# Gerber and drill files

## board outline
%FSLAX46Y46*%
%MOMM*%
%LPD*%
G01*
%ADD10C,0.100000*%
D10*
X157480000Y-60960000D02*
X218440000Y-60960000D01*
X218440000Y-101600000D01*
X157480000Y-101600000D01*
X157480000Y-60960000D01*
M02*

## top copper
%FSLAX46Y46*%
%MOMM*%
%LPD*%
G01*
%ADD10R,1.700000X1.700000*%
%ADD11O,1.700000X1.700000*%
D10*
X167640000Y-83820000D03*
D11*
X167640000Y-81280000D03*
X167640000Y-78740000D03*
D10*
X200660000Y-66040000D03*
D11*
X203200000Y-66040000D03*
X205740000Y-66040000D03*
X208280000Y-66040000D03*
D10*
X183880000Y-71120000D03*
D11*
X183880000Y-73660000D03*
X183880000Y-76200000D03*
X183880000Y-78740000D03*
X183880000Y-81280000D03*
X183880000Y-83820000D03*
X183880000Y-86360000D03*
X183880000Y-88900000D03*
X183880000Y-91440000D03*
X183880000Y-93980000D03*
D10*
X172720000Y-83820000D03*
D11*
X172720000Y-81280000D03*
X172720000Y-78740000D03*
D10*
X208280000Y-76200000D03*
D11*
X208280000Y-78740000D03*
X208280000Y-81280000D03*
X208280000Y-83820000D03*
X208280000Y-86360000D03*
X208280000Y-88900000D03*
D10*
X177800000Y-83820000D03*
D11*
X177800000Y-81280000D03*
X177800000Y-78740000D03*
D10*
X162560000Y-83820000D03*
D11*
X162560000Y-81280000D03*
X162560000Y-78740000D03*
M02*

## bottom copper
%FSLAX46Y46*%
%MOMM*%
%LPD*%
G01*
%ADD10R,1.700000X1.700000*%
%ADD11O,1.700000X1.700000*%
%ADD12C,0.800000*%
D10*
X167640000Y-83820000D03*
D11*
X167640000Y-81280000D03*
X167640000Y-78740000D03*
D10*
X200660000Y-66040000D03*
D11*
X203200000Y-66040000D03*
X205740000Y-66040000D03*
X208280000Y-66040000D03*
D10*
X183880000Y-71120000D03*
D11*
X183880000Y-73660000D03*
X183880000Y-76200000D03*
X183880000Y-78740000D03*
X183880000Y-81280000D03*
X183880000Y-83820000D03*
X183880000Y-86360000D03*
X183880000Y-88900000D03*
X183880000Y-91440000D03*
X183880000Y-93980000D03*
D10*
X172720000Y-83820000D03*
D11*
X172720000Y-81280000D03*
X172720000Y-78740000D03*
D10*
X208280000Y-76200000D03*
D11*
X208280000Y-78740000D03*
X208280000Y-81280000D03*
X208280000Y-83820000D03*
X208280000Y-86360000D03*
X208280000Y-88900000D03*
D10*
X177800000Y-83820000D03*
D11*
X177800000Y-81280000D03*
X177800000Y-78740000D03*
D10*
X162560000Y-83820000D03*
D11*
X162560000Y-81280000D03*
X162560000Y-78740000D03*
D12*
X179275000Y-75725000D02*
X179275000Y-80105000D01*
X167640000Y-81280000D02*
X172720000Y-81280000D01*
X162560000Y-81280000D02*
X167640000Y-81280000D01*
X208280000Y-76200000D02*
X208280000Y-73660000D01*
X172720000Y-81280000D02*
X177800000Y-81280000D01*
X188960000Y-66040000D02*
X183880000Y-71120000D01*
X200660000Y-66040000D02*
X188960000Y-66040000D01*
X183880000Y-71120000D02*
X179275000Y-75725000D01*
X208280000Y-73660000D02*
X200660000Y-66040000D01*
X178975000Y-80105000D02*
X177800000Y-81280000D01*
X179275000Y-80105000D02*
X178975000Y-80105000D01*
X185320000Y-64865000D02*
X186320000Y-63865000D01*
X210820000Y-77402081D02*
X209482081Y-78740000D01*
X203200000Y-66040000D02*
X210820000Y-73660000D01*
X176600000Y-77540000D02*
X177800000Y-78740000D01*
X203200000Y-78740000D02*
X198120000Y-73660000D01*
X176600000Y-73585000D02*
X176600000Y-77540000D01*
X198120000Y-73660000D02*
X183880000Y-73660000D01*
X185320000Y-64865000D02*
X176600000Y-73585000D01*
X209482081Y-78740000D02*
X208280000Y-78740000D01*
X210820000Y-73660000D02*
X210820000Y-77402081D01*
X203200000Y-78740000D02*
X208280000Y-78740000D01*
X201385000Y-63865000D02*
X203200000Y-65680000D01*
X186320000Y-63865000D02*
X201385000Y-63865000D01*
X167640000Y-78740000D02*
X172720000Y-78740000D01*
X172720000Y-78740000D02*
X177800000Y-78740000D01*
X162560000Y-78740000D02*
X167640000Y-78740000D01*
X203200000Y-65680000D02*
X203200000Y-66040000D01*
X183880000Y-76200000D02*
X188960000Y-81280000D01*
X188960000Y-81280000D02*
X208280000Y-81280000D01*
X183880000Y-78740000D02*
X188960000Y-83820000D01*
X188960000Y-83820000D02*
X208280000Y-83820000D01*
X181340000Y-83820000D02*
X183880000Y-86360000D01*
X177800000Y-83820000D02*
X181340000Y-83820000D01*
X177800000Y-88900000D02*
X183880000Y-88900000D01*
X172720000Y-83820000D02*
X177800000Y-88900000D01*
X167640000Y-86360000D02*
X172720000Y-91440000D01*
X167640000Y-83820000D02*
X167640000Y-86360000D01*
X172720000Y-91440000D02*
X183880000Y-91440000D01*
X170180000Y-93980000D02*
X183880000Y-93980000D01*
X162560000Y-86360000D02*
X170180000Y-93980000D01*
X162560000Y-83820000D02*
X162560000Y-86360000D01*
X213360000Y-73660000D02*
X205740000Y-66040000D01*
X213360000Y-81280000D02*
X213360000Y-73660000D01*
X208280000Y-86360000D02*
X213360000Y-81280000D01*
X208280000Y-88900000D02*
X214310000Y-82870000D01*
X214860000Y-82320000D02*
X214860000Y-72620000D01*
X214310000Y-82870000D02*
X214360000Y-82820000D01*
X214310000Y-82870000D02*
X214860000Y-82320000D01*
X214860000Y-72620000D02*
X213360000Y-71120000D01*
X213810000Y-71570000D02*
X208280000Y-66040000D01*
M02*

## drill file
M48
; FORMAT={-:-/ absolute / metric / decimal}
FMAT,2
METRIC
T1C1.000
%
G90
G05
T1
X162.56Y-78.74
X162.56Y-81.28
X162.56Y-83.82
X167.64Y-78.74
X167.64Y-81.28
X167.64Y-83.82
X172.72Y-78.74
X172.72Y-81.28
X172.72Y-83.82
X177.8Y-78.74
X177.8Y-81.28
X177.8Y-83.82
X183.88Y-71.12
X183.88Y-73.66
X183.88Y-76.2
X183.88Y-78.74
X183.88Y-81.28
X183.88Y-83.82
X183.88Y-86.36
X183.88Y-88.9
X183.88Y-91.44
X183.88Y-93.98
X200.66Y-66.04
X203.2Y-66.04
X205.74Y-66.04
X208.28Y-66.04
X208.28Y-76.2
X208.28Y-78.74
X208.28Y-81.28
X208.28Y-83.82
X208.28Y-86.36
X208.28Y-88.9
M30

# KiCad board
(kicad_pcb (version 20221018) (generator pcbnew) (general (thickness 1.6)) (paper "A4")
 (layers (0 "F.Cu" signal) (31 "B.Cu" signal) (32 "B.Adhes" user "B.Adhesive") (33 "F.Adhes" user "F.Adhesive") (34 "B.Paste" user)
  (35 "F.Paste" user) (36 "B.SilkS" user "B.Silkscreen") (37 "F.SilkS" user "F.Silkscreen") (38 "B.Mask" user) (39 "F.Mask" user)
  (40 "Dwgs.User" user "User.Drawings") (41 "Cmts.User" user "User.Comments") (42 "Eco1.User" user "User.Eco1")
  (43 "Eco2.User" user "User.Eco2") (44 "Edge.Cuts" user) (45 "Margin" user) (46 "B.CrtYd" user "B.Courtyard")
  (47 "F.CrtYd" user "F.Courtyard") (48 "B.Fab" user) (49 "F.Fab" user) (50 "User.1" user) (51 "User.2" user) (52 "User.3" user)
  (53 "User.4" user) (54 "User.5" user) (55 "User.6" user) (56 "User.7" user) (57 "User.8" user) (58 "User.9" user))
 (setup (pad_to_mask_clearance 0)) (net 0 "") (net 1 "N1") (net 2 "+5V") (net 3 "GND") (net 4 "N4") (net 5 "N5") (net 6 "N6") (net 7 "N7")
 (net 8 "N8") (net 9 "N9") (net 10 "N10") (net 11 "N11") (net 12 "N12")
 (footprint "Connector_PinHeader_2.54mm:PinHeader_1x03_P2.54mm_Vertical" (layer "F.Cu") (at 167.64 83.82 180)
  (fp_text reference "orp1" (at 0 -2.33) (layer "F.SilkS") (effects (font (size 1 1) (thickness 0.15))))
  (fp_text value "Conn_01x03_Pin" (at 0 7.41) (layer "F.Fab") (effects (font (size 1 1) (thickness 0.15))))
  (pad "1" thru_hole rect (at 0 0 180) (size 1.7 1.7) (drill 1) (layers "*.Cu" "*.Mask") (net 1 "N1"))
  (pad "2" thru_hole oval (at 0 2.54 180) (size 1.7 1.7) (drill 1) (layers "*.Cu" "*.Mask") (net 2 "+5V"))
  (pad "3" thru_hole oval (at 0 5.08 180) (size 1.7 1.7) (drill 1) (layers "*.Cu" "*.Mask") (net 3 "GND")))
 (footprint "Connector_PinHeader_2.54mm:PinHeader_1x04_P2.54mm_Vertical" (layer "F.Cu") (at 200.66 66.04 90)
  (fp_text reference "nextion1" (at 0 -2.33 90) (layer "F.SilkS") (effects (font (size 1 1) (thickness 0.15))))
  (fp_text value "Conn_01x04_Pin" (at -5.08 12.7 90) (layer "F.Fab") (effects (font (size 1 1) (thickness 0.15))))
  (pad "1" thru_hole rect (at 0 0 90) (size 1.7 1.7) (drill 1) (layers "*.Cu" "*.Mask") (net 2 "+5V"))
  (pad "2" thru_hole oval (at 0 2.54 90) (size 1.7 1.7) (drill 1) (layers "*.Cu" "*.Mask") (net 3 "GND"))
  (pad "3" thru_hole oval (at 0 5.08 90) (size 1.7 1.7) (drill 1) (layers "*.Cu" "*.Mask") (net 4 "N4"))
  (pad "4" thru_hole oval (at 0 7.62 90) (size 1.7 1.7) (drill 1) (layers "*.Cu" "*.Mask") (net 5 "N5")))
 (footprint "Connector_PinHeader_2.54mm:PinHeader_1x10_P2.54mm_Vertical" (layer "F.Cu") (at 183.88 71.12)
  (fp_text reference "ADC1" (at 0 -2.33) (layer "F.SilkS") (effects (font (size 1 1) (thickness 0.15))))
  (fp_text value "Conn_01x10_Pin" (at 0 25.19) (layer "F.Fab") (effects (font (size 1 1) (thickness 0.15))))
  (pad "1" thru_hole rect (at 0 0) (size 1.7 1.7) (drill 1) (layers "*.Cu" "*.Mask") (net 2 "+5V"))
  (pad "2" thru_hole oval (at 0 2.54) (size 1.7 1.7) (drill 1) (layers "*.Cu" "*.Mask") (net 3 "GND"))
  (pad "3" thru_hole oval (at 0 5.08) (size 1.7 1.7) (drill 1) (layers "*.Cu" "*.Mask") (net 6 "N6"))
  (pad "4" thru_hole oval (at 0 7.62) (size 1.7 1.7) (drill 1) (layers "*.Cu" "*.Mask") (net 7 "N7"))
  (pad "5" thru_hole oval (at 0 10.16) (size 1.7 1.7) (drill 1) (layers "*.Cu" "*.Mask") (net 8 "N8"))
  (pad "6" thru_hole oval (at 0 12.7) (size 1.7 1.7) (drill 1) (layers "*.Cu" "*.Mask") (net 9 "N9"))
  (pad "7" thru_hole oval (at 0 15.24) (size 1.7 1.7) (drill 1) (layers "*.Cu" "*.Mask") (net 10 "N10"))
  (pad "8" thru_hole oval (at 0 17.78) (size 1.7 1.7) (drill 1) (layers "*.Cu" "*.Mask") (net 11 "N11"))
  (pad "9" thru_hole oval (at 0 20.32) (size 1.7 1.7) (drill 1) (layers "*.Cu" "*.Mask") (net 1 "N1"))
  (pad "10" thru_hole oval (at 0 22.86) (size 1.7 1.7) (drill 1) (layers "*.Cu" "*.Mask") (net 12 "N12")))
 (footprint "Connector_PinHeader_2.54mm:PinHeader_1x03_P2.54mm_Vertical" (layer "F.Cu") (at 172.72 83.82 180)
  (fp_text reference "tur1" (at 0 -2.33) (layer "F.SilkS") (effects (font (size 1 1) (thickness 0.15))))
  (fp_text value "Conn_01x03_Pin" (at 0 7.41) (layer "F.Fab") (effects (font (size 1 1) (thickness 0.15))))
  (pad "1" thru_hole rect (at 0 0 180) (size 1.7 1.7) (drill 1) (layers "*.Cu" "*.Mask") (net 11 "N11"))
  (pad "2" thru_hole oval (at 0 2.54 180) (size 1.7 1.7) (drill 1) (layers "*.Cu" "*.Mask") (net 2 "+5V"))
  (pad "3" thru_hole oval (at 0 5.08 180) (size 1.7 1.7) (drill 1) (layers "*.Cu" "*.Mask") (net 3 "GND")))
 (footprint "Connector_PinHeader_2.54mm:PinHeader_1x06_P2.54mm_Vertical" (layer "F.Cu") (at 208.28 76.2)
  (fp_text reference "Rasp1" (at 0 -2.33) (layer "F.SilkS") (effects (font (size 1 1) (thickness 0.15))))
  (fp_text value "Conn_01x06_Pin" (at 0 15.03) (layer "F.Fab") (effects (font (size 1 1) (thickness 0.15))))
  (pad "1" thru_hole rect (at 0 0) (size 1.7 1.7) (drill 1) (layers "*.Cu" "*.Mask") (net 2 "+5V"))
  (pad "2" thru_hole oval (at 0 2.54) (size 1.7 1.7) (drill 1) (layers "*.Cu" "*.Mask") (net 3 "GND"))
  (pad "3" thru_hole oval (at 0 5.08) (size 1.7 1.7) (drill 1) (layers "*.Cu" "*.Mask") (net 6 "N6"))
  (pad "4" thru_hole oval (at 0 7.62) (size 1.7 1.7) (drill 1) (layers "*.Cu" "*.Mask") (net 7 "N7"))
  (pad "5" thru_hole oval (at 0 10.16) (size 1.7 1.7) (drill 1) (layers "*.Cu" "*.Mask") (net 4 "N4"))
  (pad "6" thru_hole oval (at 0 12.7) (size 1.7 1.7) (drill 1) (layers "*.Cu" "*.Mask") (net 5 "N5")))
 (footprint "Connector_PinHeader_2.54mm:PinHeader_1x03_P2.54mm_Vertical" (layer "F.Cu") (at 177.8 83.82 180)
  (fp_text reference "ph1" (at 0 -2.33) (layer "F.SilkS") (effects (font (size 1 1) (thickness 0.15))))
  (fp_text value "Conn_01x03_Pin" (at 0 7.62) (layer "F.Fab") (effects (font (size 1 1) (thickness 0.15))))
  (pad "1" thru_hole rect (at 0 0 180) (size 1.7 1.7) (drill 1) (layers "*.Cu" "*.Mask") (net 10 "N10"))
  (pad "2" thru_hole oval (at 0 2.54 180) (size 1.7 1.7) (drill 1) (layers "*.Cu" "*.Mask") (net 2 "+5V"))
  (pad "3" thru_hole oval (at 0 5.08 180) (size 1.7 1.7) (drill 1) (layers "*.Cu" "*.Mask") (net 3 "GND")))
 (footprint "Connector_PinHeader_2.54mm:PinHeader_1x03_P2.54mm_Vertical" (layer "F.Cu") (at 162.56 83.82 180)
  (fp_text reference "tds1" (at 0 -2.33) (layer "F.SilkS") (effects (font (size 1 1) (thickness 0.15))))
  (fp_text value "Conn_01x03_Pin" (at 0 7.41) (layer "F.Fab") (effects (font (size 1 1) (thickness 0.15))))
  (pad "1" thru_hole rect (at 0 0 180) (size 1.7 1.7) (drill 1) (layers "*.Cu" "*.Mask") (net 12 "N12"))
  (pad "2" thru_hole oval (at 0 2.54 180) (size 1.7 1.7) (drill 1) (layers "*.Cu" "*.Mask") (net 2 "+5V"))
  (pad "3" thru_hole oval (at 0 5.08 180) (size 1.7 1.7) (drill 1) (layers "*.Cu" "*.Mask") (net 3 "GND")))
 (gr_rect (start 157.48 60.96) (end 218.44 101.6) (stroke (width 0.1) (type default)) (fill none) (layer "Edge.Cuts"))
 (segment (start 179.275 75.725) (end 179.275 80.105) (width 0.8) (layer "B.Cu") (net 2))
 (segment (start 167.64 81.28) (end 172.72 81.28) (width 0.8) (layer "B.Cu") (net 2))
 (segment (start 162.56 81.28) (end 167.64 81.28) (width 0.8) (layer "B.Cu") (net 2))
 (segment (start 208.28 76.2) (end 208.28 73.66) (width 0.8) (layer "B.Cu") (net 2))
 (segment (start 172.72 81.28) (end 177.8 81.28) (width 0.8) (layer "B.Cu") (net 2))
 (segment (start 188.96 66.04) (end 183.88 71.12) (width 0.8) (layer "B.Cu") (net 2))
 (segment (start 200.66 66.04) (end 188.96 66.04) (width 0.8) (layer "B.Cu") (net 2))
 (segment (start 183.88 71.12) (end 179.275 75.725) (width 0.8) (layer "B.Cu") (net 2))
 (segment (start 208.28 73.66) (end 200.66 66.04) (width 0.8) (layer "B.Cu") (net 2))
 (segment (start 178.975 80.105) (end 177.8 81.28) (width 0.8) (layer "B.Cu") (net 2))
 (segment (start 179.275 80.105) (end 178.975 80.105) (width 0.8) (layer "B.Cu") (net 2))
 (segment (start 185.32 64.865) (end 186.32 63.865) (width 0.8) (layer "B.Cu") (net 3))
 (segment (start 210.82 77.402081) (end 209.482081 78.74) (width 0.8) (layer "B.Cu") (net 3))
 (segment (start 203.2 66.04) (end 210.82 73.66) (width 0.8) (layer "B.Cu") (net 3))
 (segment (start 176.6 77.54) (end 177.8 78.74) (width 0.8) (layer "B.Cu") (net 3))
 (segment (start 203.2 78.74) (end 198.12 73.66) (width 0.8) (layer "B.Cu") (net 3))
 (segment (start 176.6 73.585) (end 176.6 77.54) (width 0.8) (layer "B.Cu") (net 3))
 (segment (start 198.12 73.66) (end 183.88 73.66) (width 0.8) (layer "B.Cu") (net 3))
 (segment (start 185.32 64.865) (end 176.6 73.585) (width 0.8) (layer "B.Cu") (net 3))
 (segment (start 209.482081 78.74) (end 208.28 78.74) (width 0.8) (layer "B.Cu") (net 3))
 (segment (start 210.82 73.66) (end 210.82 77.402081) (width 0.8) (layer "B.Cu") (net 3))
 (segment (start 203.2 78.74) (end 208.28 78.74) (width 0.8) (layer "B.Cu") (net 3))
 (segment (start 201.385 63.865) (end 203.2 65.68) (width 0.8) (layer "B.Cu") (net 3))
 (segment (start 186.32 63.865) (end 201.385 63.865) (width 0.8) (layer "B.Cu") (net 3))
 (segment (start 167.64 78.74) (end 172.72 78.74) (width 0.8) (layer "B.Cu") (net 3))
 (segment (start 172.72 78.74) (end 177.8 78.74) (width 0.8) (layer "B.Cu") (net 3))
 (segment (start 162.56 78.74) (end 167.64 78.74) (width 0.8) (layer "B.Cu") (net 3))
 (segment (start 203.2 65.68) (end 203.2 66.04) (width 0.8) (layer "B.Cu") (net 3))
 (segment (start 183.88 76.2) (end 188.96 81.28) (width 0.8) (layer "B.Cu") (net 6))
 (segment (start 188.96 81.28) (end 208.28 81.28) (width 0.8) (layer "B.Cu") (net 6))
 (segment (start 183.88 78.74) (end 188.96 83.82) (width 0.8) (layer "B.Cu") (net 7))
 (segment (start 188.96 83.82) (end 208.28 83.82) (width 0.8) (layer "B.Cu") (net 7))
 (segment (start 181.34 83.82) (end 183.88 86.36) (width 0.8) (layer "B.Cu") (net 10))
 (segment (start 177.8 83.82) (end 181.34 83.82) (width 0.8) (layer "B.Cu") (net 10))
 (segment (start 177.8 88.9) (end 183.88 88.9) (width 0.8) (layer "B.Cu") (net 11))
 (segment (start 172.72 83.82) (end 177.8 88.9) (width 0.8) (layer "B.Cu") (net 11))
 (segment (start 167.64 86.36) (end 172.72 91.44) (width 0.8) (layer "B.Cu") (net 1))
 (segment (start 167.64 83.82) (end 167.64 86.36) (width 0.8) (layer "B.Cu") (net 1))
 (segment (start 172.72 91.44) (end 183.88 91.44) (width 0.8) (layer "B.Cu") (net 1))
 (segment (start 170.18 93.98) (end 183.88 93.98) (width 0.8) (layer "B.Cu") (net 12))
 (segment (start 162.56 86.36) (end 170.18 93.98) (width 0.8) (layer "B.Cu") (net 12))
 (segment (start 162.56 83.82) (end 162.56 86.36) (width 0.8) (layer "B.Cu") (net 12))
 (segment (start 213.36 73.66) (end 205.74 66.04) (width 0.8) (layer "B.Cu") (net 4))
 (segment (start 213.36 81.28) (end 213.36 73.66) (width 0.8) (layer "B.Cu") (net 4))
 (segment (start 208.28 86.36) (end 213.36 81.28) (width 0.8) (layer "B.Cu") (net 4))
 (segment (start 208.28 88.9) (end 214.31 82.87) (width 0.8) (layer "B.Cu") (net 5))
 (segment (start 214.86 82.32) (end 214.86 72.62) (width 0.8) (layer "B.Cu") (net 5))
 (segment (start 214.31 82.87) (end 214.36 82.82) (width 0.8) (layer "B.Cu") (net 5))
 (segment (start 214.31 82.87) (end 214.86 82.32) (width 0.8) (layer "B.Cu") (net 5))
 (segment (start 214.86 72.62) (end 213.36 71.12) (width 0.8) (layer "B.Cu") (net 5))
 (segment (start 213.81 71.57) (end 208.28 66.04) (width 0.8) (layer "B.Cu") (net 5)))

